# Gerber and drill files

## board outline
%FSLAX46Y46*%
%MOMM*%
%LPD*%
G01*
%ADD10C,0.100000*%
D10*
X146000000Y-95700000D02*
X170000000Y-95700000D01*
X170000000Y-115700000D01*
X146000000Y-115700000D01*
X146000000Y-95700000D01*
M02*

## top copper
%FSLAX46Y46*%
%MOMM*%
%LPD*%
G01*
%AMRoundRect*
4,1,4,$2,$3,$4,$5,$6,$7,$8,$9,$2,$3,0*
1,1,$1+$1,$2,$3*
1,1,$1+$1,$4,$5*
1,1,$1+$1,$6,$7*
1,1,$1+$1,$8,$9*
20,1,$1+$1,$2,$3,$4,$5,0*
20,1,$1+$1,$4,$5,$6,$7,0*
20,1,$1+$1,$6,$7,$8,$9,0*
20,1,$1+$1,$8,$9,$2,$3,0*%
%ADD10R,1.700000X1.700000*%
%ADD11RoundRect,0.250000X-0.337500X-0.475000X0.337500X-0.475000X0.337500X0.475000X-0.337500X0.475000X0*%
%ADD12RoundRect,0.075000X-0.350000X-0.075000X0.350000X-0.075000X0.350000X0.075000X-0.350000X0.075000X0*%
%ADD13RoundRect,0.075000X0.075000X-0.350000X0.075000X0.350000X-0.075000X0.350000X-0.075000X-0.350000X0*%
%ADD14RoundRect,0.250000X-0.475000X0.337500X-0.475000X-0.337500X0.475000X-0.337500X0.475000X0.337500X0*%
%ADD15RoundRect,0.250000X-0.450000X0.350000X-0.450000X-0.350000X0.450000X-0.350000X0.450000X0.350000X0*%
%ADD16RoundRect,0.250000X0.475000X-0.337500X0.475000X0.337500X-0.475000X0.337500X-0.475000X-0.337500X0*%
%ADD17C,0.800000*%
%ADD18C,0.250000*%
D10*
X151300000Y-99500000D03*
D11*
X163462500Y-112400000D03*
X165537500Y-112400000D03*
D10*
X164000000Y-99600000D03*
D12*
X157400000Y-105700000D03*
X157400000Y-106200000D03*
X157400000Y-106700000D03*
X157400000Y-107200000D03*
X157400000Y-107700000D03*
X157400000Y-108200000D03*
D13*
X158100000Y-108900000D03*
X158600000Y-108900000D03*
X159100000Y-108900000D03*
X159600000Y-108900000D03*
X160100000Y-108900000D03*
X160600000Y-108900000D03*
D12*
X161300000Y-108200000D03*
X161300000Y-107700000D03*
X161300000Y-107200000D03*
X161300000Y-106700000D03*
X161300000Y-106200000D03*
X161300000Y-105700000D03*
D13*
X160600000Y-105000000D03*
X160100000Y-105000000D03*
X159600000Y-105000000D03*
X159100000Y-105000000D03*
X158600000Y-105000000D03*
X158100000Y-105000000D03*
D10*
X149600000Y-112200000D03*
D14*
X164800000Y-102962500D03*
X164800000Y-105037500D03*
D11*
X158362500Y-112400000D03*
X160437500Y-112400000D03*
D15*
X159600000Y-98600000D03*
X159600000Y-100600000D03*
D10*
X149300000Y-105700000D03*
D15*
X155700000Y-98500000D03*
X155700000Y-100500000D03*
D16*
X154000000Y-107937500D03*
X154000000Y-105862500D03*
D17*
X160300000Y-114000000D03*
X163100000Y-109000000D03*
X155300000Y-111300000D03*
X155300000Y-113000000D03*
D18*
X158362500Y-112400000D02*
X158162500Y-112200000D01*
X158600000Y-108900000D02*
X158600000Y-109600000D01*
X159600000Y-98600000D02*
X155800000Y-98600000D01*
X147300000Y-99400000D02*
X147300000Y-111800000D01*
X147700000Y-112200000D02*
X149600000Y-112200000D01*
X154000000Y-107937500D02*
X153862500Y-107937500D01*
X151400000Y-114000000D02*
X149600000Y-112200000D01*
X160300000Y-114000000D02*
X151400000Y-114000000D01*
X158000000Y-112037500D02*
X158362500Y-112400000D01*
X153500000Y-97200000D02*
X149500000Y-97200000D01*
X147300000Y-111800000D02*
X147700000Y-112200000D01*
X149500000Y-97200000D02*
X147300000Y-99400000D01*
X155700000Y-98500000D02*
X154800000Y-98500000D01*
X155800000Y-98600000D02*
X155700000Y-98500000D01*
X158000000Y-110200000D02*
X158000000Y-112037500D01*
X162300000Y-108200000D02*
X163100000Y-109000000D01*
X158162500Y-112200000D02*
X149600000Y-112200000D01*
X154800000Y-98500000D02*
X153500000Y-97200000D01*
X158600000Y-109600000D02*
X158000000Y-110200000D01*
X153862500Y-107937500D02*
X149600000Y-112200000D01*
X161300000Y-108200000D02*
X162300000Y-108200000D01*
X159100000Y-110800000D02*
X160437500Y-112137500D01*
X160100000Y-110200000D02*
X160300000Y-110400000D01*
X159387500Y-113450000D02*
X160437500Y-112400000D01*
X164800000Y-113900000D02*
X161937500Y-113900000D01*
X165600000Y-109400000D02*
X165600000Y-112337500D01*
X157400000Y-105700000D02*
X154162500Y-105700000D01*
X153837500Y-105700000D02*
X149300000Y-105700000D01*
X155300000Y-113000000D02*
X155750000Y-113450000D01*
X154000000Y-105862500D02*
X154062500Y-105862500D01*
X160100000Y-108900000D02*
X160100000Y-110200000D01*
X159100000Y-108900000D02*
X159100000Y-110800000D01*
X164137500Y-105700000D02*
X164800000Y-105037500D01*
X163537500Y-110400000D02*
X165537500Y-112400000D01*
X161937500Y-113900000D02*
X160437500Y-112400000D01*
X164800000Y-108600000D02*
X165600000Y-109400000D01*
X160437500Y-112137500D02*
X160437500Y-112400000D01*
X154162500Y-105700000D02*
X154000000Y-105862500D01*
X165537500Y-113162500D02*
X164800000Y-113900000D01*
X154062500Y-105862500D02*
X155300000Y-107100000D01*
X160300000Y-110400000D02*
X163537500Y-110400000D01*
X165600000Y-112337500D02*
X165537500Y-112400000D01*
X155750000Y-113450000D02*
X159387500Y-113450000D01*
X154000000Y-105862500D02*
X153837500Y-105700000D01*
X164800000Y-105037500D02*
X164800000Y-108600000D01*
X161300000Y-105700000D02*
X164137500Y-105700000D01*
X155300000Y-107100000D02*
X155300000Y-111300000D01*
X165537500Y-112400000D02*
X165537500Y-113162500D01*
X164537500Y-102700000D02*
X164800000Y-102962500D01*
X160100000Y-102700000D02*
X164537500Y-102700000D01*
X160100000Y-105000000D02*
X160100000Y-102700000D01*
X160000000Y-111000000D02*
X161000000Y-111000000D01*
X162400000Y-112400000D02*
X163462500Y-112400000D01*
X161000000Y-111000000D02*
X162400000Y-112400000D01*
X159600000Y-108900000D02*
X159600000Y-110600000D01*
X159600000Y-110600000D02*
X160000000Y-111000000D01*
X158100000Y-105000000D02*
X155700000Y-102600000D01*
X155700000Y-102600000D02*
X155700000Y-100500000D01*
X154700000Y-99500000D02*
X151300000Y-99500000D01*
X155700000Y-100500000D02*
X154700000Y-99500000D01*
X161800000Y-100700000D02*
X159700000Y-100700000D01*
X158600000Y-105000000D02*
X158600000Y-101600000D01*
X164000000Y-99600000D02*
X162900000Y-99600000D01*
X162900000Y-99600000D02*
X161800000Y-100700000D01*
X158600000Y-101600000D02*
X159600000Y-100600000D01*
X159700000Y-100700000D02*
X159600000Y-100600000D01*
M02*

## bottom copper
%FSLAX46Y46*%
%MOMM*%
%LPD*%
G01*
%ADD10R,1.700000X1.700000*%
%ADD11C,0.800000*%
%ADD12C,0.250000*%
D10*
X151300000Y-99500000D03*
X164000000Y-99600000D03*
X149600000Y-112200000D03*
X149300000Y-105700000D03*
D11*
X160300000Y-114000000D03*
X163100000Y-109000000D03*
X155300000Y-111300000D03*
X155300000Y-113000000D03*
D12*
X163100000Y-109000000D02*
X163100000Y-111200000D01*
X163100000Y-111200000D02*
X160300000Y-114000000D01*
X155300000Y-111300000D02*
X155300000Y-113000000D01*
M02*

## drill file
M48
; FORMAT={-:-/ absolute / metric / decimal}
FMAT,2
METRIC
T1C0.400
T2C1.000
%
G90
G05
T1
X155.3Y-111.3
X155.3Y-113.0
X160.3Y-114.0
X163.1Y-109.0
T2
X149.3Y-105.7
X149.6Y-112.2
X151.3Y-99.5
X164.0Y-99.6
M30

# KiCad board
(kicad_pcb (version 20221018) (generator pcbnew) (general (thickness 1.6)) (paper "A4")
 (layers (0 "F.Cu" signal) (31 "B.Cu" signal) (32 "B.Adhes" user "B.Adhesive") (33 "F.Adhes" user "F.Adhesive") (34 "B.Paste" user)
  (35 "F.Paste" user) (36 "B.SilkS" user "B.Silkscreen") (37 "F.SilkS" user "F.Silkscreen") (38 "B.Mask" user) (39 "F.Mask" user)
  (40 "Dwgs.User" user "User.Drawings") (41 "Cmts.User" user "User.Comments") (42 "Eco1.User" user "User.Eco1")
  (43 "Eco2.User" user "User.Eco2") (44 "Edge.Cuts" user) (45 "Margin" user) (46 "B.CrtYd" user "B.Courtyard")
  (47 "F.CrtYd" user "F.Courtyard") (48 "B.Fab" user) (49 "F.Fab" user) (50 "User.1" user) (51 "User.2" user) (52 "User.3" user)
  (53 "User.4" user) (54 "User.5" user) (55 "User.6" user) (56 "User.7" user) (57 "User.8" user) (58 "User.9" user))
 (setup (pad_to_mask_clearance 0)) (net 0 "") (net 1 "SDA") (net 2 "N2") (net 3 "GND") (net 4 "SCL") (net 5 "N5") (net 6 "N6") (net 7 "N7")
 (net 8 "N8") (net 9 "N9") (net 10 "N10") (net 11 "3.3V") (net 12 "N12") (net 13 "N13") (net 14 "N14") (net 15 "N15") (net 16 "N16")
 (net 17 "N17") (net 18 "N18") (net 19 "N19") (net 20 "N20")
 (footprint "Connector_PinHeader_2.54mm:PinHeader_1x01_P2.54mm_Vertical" (layer "F.Cu") (at 151.3 99.5)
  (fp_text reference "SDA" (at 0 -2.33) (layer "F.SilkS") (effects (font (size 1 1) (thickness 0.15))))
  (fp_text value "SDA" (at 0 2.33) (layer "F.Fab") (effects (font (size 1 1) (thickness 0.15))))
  (pad "1" thru_hole rect (at 0 0) (size 1.7 1.7) (drill 1) (layers "*.Cu" "*.Mask") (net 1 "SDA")))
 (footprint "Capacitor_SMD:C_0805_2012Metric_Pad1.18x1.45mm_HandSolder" (layer "F.Cu") (at 164.5 112.4)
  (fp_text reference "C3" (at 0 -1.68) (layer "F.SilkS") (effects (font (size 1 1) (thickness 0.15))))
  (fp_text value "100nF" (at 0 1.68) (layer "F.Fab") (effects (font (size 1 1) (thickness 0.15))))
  (pad "1" smd roundrect (at -1.0375 0) (size 1.175 1.45) (layers "F.Cu" "F.Paste" "F.Mask") (roundrect_rratio 0.212766) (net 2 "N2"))
  (pad "2" smd roundrect (at 1.0375 0) (size 1.175 1.45) (layers "F.Cu" "F.Paste" "F.Mask") (roundrect_rratio 0.212766) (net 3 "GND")))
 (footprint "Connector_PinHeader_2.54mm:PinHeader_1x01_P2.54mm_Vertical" (layer "F.Cu") (at 164 99.6)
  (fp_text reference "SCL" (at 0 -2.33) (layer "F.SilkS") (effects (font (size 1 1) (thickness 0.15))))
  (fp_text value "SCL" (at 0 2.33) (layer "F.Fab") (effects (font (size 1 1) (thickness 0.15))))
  (pad "1" thru_hole rect (at 0 0) (size 1.7 1.7) (drill 1) (layers "*.Cu" "*.Mask") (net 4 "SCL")))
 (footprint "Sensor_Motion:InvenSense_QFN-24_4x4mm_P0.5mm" (layer "F.Cu") (at 159.35 106.95)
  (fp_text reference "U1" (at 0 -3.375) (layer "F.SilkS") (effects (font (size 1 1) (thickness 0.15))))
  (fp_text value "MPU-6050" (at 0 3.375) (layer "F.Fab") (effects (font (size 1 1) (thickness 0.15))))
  (pad "1" smd roundrect (at -1.95 -1.25) (size 0.85 0.3) (layers "F.Cu" "F.Paste" "F.Mask") (roundrect_rratio 0.25) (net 3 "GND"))
  (pad "2" smd roundrect (at -1.95 -0.75) (size 0.85 0.3) (layers "F.Cu" "F.Paste" "F.Mask") (roundrect_rratio 0.25) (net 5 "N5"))
  (pad "3" smd roundrect (at -1.95 -0.25) (size 0.85 0.3) (layers "F.Cu" "F.Paste" "F.Mask") (roundrect_rratio 0.25) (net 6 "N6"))
  (pad "4" smd roundrect (at -1.95 0.25) (size 0.85 0.3) (layers "F.Cu" "F.Paste" "F.Mask") (roundrect_rratio 0.25) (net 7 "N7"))
  (pad "5" smd roundrect (at -1.95 0.75) (size 0.85 0.3) (layers "F.Cu" "F.Paste" "F.Mask") (roundrect_rratio 0.25) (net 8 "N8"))
  (pad "6" smd roundrect (at -1.95 1.25) (size 0.85 0.3) (layers "F.Cu" "F.Paste" "F.Mask") (roundrect_rratio 0.25) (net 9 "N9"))
  (pad "7" smd roundrect (at -1.25 1.95 90) (size 0.85 0.3) (layers "F.Cu" "F.Paste" "F.Mask") (roundrect_rratio 0.25) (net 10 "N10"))
  (pad "8" smd roundrect (at -0.75 1.95 90) (size 0.85 0.3) (layers "F.Cu" "F.Paste" "F.Mask") (roundrect_rratio 0.25) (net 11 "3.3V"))
  (pad "9" smd roundrect (at -0.25 1.95 90) (size 0.85 0.3) (layers "F.Cu" "F.Paste" "F.Mask") (roundrect_rratio 0.25) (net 3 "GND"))
  (pad "10" smd roundrect (at 0.25 1.95 90) (size 0.85 0.3) (layers "F.Cu" "F.Paste" "F.Mask") (roundrect_rratio 0.25) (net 2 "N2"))
  (pad "11" smd roundrect (at 0.75 1.95 90) (size 0.85 0.3) (layers "F.Cu" "F.Paste" "F.Mask") (roundrect_rratio 0.25) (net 3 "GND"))
  (pad "12" smd roundrect (at 1.25 1.95 90) (size 0.85 0.3) (layers "F.Cu" "F.Paste" "F.Mask") (roundrect_rratio 0.25) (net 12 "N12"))
  (pad "13" smd roundrect (at 1.95 1.25) (size 0.85 0.3) (layers "F.Cu" "F.Paste" "F.Mask") (roundrect_rratio 0.25) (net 11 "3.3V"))
  (pad "14" smd roundrect (at 1.95 0.75) (size 0.85 0.3) (layers "F.Cu" "F.Paste" "F.Mask") (roundrect_rratio 0.25) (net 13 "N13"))
  (pad "15" smd roundrect (at 1.95 0.25) (size 0.85 0.3) (layers "F.Cu" "F.Paste" "F.Mask") (roundrect_rratio 0.25) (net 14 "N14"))
  (pad "16" smd roundrect (at 1.95 -0.25) (size 0.85 0.3) (layers "F.Cu" "F.Paste" "F.Mask") (roundrect_rratio 0.25) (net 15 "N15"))
  (pad "17" smd roundrect (at 1.95 -0.75) (size 0.85 0.3) (layers "F.Cu" "F.Paste" "F.Mask") (roundrect_rratio 0.25) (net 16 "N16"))
  (pad "18" smd roundrect (at 1.95 -1.25) (size 0.85 0.3) (layers "F.Cu" "F.Paste" "F.Mask") (roundrect_rratio 0.25) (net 3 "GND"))
  (pad "19" smd roundrect (at 1.25 -1.95 90) (size 0.85 0.3) (layers "F.Cu" "F.Paste" "F.Mask") (roundrect_rratio 0.25) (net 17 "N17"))
  (pad "20" smd roundrect (at 0.75 -1.95 90) (size 0.85 0.3) (layers "F.Cu" "F.Paste" "F.Mask") (roundrect_rratio 0.25) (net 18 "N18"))
  (pad "21" smd roundrect (at 0.25 -1.95 90) (size 0.85 0.3) (layers "F.Cu" "F.Paste" "F.Mask") (roundrect_rratio 0.25) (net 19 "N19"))
  (pad "22" smd roundrect (at -0.25 -1.95 90) (size 0.85 0.3) (layers "F.Cu" "F.Paste" "F.Mask") (roundrect_rratio 0.25) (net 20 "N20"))
  (pad "23" smd roundrect (at -0.75 -1.95 90) (size 0.85 0.3) (layers "F.Cu" "F.Paste" "F.Mask") (roundrect_rratio 0.25) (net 4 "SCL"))
  (pad "24" smd roundrect (at -1.25 -1.95 90) (size 0.85 0.3) (layers "F.Cu" "F.Paste" "F.Mask") (roundrect_rratio 0.25) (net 1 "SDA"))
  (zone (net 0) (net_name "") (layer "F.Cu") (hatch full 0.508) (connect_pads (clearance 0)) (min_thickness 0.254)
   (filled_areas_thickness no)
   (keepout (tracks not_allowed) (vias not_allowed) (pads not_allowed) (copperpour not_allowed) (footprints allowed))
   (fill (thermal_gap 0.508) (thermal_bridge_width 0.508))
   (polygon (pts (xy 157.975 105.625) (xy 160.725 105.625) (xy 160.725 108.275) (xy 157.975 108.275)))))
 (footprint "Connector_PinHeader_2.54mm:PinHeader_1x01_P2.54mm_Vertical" (layer "F.Cu") (at 149.6 112.2)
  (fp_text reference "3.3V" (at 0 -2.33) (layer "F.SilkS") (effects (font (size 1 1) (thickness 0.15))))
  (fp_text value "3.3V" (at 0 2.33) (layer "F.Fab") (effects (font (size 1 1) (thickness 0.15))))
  (pad "1" thru_hole rect (at 0 0) (size 1.7 1.7) (drill 1) (layers "*.Cu" "*.Mask") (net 11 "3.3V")))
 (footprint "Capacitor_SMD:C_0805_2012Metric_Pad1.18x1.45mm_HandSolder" (layer "F.Cu") (at 164.8 104 -90)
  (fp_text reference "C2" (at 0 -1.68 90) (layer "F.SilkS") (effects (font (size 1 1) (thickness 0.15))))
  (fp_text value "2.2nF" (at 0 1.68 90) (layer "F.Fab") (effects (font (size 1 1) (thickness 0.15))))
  (pad "1" smd roundrect (at -1.0375 0 270) (size 1.175 1.45) (layers "F.Cu" "F.Paste" "F.Mask") (roundrect_rratio 0.212766) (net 18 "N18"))
  (pad "2" smd roundrect (at 1.0375 0 270) (size 1.175 1.45) (layers "F.Cu" "F.Paste" "F.Mask") (roundrect_rratio 0.212766) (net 3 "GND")))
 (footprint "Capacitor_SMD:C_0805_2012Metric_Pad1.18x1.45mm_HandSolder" (layer "F.Cu") (at 159.4 112.4)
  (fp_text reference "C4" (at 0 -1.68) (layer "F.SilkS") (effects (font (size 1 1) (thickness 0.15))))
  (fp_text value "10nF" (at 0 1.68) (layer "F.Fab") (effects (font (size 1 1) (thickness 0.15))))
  (pad "1" smd roundrect (at -1.0375 0) (size 1.175 1.45) (layers "F.Cu" "F.Paste" "F.Mask") (roundrect_rratio 0.212766) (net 11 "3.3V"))
  (pad "2" smd roundrect (at 1.0375 0) (size 1.175 1.45) (layers "F.Cu" "F.Paste" "F.Mask") (roundrect_rratio 0.212766) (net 3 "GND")))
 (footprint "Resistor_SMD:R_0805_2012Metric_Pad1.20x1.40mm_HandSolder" (layer "F.Cu") (at 159.6 99.6 -90)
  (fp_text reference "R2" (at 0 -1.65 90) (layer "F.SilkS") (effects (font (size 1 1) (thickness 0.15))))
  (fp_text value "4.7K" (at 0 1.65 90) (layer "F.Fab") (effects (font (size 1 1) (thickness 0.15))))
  (pad "1" smd roundrect (at -1 0 270) (size 1.2 1.4) (layers "F.Cu" "F.Paste" "F.Mask") (roundrect_rratio 0.208333) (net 11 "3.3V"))
  (pad "2" smd roundrect (at 1 0 270) (size 1.2 1.4) (layers "F.Cu" "F.Paste" "F.Mask") (roundrect_rratio 0.208333) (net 4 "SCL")))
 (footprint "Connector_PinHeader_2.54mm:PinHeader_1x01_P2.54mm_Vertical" (layer "F.Cu") (at 149.3 105.7)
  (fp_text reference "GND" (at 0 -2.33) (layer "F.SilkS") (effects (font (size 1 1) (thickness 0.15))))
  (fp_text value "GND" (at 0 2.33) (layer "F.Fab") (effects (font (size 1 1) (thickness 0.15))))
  (pad "1" thru_hole rect (at 0 0) (size 1.7 1.7) (drill 1) (layers "*.Cu" "*.Mask") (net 3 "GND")))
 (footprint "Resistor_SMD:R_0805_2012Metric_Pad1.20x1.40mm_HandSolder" (layer "F.Cu") (at 155.7 99.5 -90)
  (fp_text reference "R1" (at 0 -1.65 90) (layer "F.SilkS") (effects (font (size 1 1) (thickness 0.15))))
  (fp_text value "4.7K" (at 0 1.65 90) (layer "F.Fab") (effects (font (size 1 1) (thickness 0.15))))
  (pad "1" smd roundrect (at -1 0 270) (size 1.2 1.4) (layers "F.Cu" "F.Paste" "F.Mask") (roundrect_rratio 0.208333) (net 11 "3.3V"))
  (pad "2" smd roundrect (at 1 0 270) (size 1.2 1.4) (layers "F.Cu" "F.Paste" "F.Mask") (roundrect_rratio 0.208333) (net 1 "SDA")))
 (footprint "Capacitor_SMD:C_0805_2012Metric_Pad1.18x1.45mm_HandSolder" (layer "F.Cu") (at 154 106.9 90)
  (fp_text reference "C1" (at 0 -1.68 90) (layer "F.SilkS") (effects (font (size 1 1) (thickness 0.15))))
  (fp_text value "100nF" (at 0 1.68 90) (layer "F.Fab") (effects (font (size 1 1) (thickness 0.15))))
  (pad "1" smd roundrect (at -1.0375 0 90) (size 1.175 1.45) (layers "F.Cu" "F.Paste" "F.Mask") (roundrect_rratio 0.212766) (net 11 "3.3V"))
  (pad "2" smd roundrect (at 1.0375 0 90) (size 1.175 1.45) (layers "F.Cu" "F.Paste" "F.Mask") (roundrect_rratio 0.212766) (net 3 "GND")))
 (gr_rect (start 146 95.7) (end 170 115.7) (stroke (width 0.1) (type default)) (fill none) (layer "Edge.Cuts"))
 (segment (start 158.3625 112.4) (end 158.1625 112.2) (width 0.25) (layer "F.Cu") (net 11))
 (segment (start 158.6 108.9) (end 158.6 109.6) (width 0.25) (layer "F.Cu") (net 11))
 (segment (start 159.6 98.6) (end 155.8 98.6) (width 0.25) (layer "F.Cu") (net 11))
 (segment (start 147.3 99.4) (end 147.3 111.8) (width 0.25) (layer "F.Cu") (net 11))
 (segment (start 147.7 112.2) (end 149.6 112.2) (width 0.25) (layer "F.Cu") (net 11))
 (segment (start 154 107.9375) (end 153.8625 107.9375) (width 0.25) (layer "F.Cu") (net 11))
 (segment (start 151.4 114) (end 149.6 112.2) (width 0.25) (layer "F.Cu") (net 11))
 (segment (start 160.3 114) (end 151.4 114) (width 0.25) (layer "F.Cu") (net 11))
 (segment (start 158 112.0375) (end 158.3625 112.4) (width 0.25) (layer "F.Cu") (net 11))
 (segment (start 153.5 97.2) (end 149.5 97.2) (width 0.25) (layer "F.Cu") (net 11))
 (segment (start 147.3 111.8) (end 147.7 112.2) (width 0.25) (layer "F.Cu") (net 11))
 (segment (start 149.5 97.2) (end 147.3 99.4) (width 0.25) (layer "F.Cu") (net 11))
 (segment (start 155.7 98.5) (end 154.8 98.5) (width 0.25) (layer "F.Cu") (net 11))
 (segment (start 155.8 98.6) (end 155.7 98.5) (width 0.25) (layer "F.Cu") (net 11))
 (segment (start 158 110.2) (end 158 112.0375) (width 0.25) (layer "F.Cu") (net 11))
 (segment (start 162.3 108.2) (end 163.1 109) (width 0.25) (layer "F.Cu") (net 11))
 (segment (start 158.1625 112.2) (end 149.6 112.2) (width 0.25) (layer "F.Cu") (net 11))
 (segment (start 154.8 98.5) (end 153.5 97.2) (width 0.25) (layer "F.Cu") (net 11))
 (segment (start 158.6 109.6) (end 158 110.2) (width 0.25) (layer "F.Cu") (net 11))
 (segment (start 153.8625 107.9375) (end 149.6 112.2) (width 0.25) (layer "F.Cu") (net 11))
 (segment (start 161.3 108.2) (end 162.3 108.2) (width 0.25) (layer "F.Cu") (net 11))
 (via (at 160.3 114) (size 0.8) (drill 0.4) (layers "F.Cu" "B.Cu") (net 11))
 (via (at 163.1 109) (size 0.8) (drill 0.4) (layers "F.Cu" "B.Cu") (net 11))
 (segment (start 163.1 109) (end 163.1 111.2) (width 0.25) (layer "B.Cu") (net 11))
 (segment (start 163.1 111.2) (end 160.3 114) (width 0.25) (layer "B.Cu") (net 11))
 (segment (start 159.1 110.8) (end 160.4375 112.1375) (width 0.25) (layer "F.Cu") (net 3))
 (segment (start 160.1 110.2) (end 160.3 110.4) (width 0.25) (layer "F.Cu") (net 3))
 (segment (start 159.3875 113.45) (end 160.4375 112.4) (width 0.25) (layer "F.Cu") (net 3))
 (segment (start 164.8 113.9) (end 161.9375 113.9) (width 0.25) (layer "F.Cu") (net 3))
 (segment (start 165.6 109.4) (end 165.6 112.3375) (width 0.25) (layer "F.Cu") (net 3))
 (segment (start 157.4 105.7) (end 154.1625 105.7) (width 0.25) (layer "F.Cu") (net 3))
 (segment (start 153.8375 105.7) (end 149.3 105.7) (width 0.25) (layer "F.Cu") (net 3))
 (segment (start 155.3 113) (end 155.75 113.45) (width 0.25) (layer "F.Cu") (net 3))
 (segment (start 154 105.8625) (end 154.0625 105.8625) (width 0.25) (layer "F.Cu") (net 3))
 (segment (start 160.1 108.9) (end 160.1 110.2) (width 0.25) (layer "F.Cu") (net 3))
 (segment (start 159.1 108.9) (end 159.1 110.8) (width 0.25) (layer "F.Cu") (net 3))
 (segment (start 164.1375 105.7) (end 164.8 105.0375) (width 0.25) (layer "F.Cu") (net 3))
 (segment (start 163.5375 110.4) (end 165.5375 112.4) (width 0.25) (layer "F.Cu") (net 3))
 (segment (start 161.9375 113.9) (end 160.4375 112.4) (width 0.25) (layer "F.Cu") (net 3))
 (segment (start 164.8 108.6) (end 165.6 109.4) (width 0.25) (layer "F.Cu") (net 3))
 (segment (start 160.4375 112.1375) (end 160.4375 112.4) (width 0.25) (layer "F.Cu") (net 3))
 (segment (start 154.1625 105.7) (end 154 105.8625) (width 0.25) (layer "F.Cu") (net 3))
 (segment (start 165.5375 113.1625) (end 164.8 113.9) (width 0.25) (layer "F.Cu") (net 3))
 (segment (start 154.0625 105.8625) (end 155.3 107.1) (width 0.25) (layer "F.Cu") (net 3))
 (segment (start 160.3 110.4) (end 163.5375 110.4) (width 0.25) (layer "F.Cu") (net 3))
 (segment (start 165.6 112.3375) (end 165.5375 112.4) (width 0.25) (layer "F.Cu") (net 3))
 (segment (start 155.75 113.45) (end 159.3875 113.45) (width 0.25) (layer "F.Cu") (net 3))
 (segment (start 154 105.8625) (end 153.8375 105.7) (width 0.25) (layer "F.Cu") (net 3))
 (segment (start 164.8 105.0375) (end 164.8 108.6) (width 0.25) (layer "F.Cu") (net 3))
 (segment (start 161.3 105.7) (end 164.1375 105.7) (width 0.25) (layer "F.Cu") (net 3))
 (segment (start 155.3 107.1) (end 155.3 111.3) (width 0.25) (layer "F.Cu") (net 3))
 (segment (start 165.5375 112.4) (end 165.5375 113.1625) (width 0.25) (layer "F.Cu") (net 3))
 (via (at 155.3 111.3) (size 0.8) (drill 0.4) (layers "F.Cu" "B.Cu") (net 3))
 (via (at 155.3 113) (size 0.8) (drill 0.4) (layers "F.Cu" "B.Cu") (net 3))
 (segment (start 155.3 111.3) (end 155.3 113) (width 0.25) (layer "B.Cu") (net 3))
 (segment (start 164.5375 102.7) (end 164.8 102.9625) (width 0.25) (layer "F.Cu") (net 18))
 (segment (start 160.1 102.7) (end 164.5375 102.7) (width 0.25) (layer "F.Cu") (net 18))
 (segment (start 160.1 105) (end 160.1 102.7) (width 0.25) (layer "F.Cu") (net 18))
 (segment (start 160 111) (end 161 111) (width 0.25) (layer "F.Cu") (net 2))
 (segment (start 162.4 112.4) (end 163.4625 112.4) (width 0.25) (layer "F.Cu") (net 2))
 (segment (start 161 111) (end 162.4 112.4) (width 0.25) (layer "F.Cu") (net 2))
 (segment (start 159.6 108.9) (end 159.6 110.6) (width 0.25) (layer "F.Cu") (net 2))
 (segment (start 159.6 110.6) (end 160 111) (width 0.25) (layer "F.Cu") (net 2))
 (segment (start 158.1 105) (end 155.7 102.6) (width 0.25) (layer "F.Cu") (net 1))
 (segment (start 155.7 102.6) (end 155.7 100.5) (width 0.25) (layer "F.Cu") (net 1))
 (segment (start 154.7 99.5) (end 151.3 99.5) (width 0.25) (layer "F.Cu") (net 1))
 (segment (start 155.7 100.5) (end 154.7 99.5) (width 0.25) (layer "F.Cu") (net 1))
 (segment (start 161.8 100.7) (end 159.7 100.7) (width 0.25) (layer "F.Cu") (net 4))
 (segment (start 158.6 105) (end 158.6 101.6) (width 0.25) (layer "F.Cu") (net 4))
 (segment (start 164 99.6) (end 162.9 99.6) (width 0.25) (layer "F.Cu") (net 4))
 (segment (start 162.9 99.6) (end 161.8 100.7) (width 0.25) (layer "F.Cu") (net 4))
 (segment (start 158.6 101.6) (end 159.6 100.6) (width 0.25) (layer "F.Cu") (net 4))
 (segment (start 159.7 100.7) (end 159.6 100.6) (width 0.25) (layer "F.Cu") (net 4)))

